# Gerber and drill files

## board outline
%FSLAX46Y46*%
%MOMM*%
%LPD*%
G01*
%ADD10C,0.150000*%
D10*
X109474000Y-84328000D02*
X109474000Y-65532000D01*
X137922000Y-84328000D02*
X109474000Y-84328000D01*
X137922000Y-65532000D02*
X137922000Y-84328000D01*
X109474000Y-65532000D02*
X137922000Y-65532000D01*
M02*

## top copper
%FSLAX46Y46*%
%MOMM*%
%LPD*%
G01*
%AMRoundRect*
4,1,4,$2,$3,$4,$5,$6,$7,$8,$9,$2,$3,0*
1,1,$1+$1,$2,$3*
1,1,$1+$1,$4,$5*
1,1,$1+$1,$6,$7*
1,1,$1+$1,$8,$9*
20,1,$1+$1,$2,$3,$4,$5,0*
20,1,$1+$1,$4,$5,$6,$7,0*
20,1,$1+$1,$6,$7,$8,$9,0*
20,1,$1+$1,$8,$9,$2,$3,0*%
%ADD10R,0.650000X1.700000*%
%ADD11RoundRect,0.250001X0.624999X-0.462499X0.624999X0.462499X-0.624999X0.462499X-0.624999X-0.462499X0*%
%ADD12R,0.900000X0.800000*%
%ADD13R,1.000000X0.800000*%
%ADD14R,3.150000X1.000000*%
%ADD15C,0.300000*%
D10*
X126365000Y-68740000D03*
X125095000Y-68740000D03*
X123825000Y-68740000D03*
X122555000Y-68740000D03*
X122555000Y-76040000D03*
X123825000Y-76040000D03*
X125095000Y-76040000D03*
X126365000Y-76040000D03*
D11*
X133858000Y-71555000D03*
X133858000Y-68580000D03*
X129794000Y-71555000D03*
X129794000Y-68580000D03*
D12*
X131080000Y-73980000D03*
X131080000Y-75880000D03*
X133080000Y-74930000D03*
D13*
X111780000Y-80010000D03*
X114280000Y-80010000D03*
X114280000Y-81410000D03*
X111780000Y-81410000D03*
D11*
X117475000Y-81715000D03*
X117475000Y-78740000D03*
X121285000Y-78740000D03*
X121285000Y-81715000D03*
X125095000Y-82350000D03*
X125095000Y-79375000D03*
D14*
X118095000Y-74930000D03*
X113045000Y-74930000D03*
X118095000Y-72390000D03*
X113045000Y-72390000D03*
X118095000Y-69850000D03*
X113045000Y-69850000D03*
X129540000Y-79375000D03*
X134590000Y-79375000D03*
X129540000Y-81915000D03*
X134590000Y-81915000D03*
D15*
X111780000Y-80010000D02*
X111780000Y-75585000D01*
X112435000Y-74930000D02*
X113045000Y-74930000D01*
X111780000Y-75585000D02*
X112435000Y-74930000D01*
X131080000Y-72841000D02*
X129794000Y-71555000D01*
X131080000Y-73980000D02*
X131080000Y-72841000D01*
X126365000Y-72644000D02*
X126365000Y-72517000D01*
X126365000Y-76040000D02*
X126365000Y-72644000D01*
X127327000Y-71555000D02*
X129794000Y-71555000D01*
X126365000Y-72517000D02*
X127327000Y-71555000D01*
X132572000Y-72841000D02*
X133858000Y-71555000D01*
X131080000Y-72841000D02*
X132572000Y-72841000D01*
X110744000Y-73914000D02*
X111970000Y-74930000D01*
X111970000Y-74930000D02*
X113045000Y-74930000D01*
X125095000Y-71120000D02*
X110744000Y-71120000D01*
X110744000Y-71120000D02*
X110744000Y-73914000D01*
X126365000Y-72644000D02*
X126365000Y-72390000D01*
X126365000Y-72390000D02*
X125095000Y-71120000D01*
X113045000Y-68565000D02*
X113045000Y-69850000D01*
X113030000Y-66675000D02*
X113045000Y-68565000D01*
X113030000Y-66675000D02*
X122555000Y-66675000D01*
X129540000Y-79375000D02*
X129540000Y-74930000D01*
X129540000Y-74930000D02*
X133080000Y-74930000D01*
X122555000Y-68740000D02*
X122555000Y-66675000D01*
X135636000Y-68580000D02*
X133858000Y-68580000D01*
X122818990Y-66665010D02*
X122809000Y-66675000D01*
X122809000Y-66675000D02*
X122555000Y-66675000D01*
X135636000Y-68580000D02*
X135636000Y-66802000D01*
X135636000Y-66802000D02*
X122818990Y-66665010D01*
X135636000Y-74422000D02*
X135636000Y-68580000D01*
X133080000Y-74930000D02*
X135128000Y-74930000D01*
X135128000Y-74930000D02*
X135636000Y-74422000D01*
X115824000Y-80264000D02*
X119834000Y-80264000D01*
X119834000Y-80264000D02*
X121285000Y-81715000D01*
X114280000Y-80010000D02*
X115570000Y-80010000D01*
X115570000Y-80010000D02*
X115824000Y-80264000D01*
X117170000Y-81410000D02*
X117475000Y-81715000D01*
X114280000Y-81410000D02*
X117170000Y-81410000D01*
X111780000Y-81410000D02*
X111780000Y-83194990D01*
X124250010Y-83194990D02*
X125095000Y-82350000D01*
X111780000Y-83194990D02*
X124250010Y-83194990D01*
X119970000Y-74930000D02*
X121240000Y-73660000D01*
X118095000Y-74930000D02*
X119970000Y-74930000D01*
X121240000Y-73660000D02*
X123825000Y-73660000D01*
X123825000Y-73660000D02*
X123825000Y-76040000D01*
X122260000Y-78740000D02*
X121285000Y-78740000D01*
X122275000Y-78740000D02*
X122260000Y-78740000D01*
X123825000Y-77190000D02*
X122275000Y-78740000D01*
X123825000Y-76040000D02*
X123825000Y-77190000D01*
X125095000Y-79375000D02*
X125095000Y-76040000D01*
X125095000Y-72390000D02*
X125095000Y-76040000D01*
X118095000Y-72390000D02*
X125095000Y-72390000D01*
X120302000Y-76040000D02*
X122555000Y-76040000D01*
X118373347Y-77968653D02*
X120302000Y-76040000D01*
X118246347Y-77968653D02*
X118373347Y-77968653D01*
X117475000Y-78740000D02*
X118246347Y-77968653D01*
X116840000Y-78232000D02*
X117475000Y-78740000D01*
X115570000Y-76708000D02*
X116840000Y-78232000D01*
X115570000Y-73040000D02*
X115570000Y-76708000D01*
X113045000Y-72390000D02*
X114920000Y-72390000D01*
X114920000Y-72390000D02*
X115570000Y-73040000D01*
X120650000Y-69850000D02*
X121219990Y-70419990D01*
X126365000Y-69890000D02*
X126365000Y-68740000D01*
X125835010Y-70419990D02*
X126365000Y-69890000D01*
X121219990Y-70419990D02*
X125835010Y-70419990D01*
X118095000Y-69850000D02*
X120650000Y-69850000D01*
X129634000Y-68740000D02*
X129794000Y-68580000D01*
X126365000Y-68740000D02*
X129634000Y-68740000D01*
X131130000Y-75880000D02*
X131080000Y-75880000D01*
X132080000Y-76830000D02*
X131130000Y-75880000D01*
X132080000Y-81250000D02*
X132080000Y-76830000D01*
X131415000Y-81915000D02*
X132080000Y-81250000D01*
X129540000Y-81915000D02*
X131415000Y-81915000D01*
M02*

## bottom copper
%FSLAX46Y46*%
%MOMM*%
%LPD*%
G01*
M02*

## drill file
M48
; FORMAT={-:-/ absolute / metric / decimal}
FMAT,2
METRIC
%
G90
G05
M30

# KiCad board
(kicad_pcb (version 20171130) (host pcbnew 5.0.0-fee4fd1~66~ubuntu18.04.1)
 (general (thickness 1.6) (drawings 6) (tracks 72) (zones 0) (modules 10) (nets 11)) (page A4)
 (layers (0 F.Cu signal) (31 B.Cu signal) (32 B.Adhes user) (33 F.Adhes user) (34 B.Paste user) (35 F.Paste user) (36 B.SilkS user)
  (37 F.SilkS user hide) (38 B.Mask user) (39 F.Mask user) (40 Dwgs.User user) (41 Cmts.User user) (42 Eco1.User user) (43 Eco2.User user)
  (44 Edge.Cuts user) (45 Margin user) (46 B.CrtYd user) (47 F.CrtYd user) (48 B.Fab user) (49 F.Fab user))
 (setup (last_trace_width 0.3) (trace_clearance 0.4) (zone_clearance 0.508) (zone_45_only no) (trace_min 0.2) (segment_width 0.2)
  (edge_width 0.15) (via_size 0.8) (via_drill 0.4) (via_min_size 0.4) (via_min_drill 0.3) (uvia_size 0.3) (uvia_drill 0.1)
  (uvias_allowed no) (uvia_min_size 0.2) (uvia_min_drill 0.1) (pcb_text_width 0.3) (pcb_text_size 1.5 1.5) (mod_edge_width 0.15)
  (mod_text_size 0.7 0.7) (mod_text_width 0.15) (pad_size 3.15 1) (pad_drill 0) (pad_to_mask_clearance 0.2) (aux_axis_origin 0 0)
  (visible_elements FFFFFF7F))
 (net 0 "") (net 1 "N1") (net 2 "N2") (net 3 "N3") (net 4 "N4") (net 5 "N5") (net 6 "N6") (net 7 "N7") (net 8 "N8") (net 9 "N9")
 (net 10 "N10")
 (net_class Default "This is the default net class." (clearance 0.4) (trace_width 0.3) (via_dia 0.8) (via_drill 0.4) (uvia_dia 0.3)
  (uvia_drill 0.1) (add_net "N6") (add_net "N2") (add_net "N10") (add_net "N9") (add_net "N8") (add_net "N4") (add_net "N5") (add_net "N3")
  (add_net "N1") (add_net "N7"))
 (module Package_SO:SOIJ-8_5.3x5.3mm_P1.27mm (layer F.Cu) (at 124.46 72.39 270)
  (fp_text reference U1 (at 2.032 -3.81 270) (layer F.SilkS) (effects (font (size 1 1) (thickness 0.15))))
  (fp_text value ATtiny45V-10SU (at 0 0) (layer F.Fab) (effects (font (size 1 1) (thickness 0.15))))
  (pad 1 smd rect (at -3.65 -1.905 270) (size 1.7 0.65) (layers F.Cu F.Paste F.Mask) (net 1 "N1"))
  (pad 2 smd rect (at -3.65 -0.635 270) (size 1.7 0.65) (layers F.Cu F.Paste F.Mask))
  (pad 3 smd rect (at -3.65 0.635 270) (size 1.7 0.65) (layers F.Cu F.Paste F.Mask))
  (pad 4 smd rect (at -3.65 1.905 270) (size 1.7 0.65) (layers F.Cu F.Paste F.Mask) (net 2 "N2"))
  (pad 5 smd rect (at 3.65 1.905 270) (size 1.7 0.65) (layers F.Cu F.Paste F.Mask) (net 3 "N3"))
  (pad 6 smd rect (at 3.65 0.635 270) (size 1.7 0.65) (layers F.Cu F.Paste F.Mask) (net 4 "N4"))
  (pad 7 smd rect (at 3.65 -0.635 270) (size 1.7 0.65) (layers F.Cu F.Paste F.Mask) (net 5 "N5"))
  (pad 8 smd rect (at 3.65 -1.905 270) (size 1.7 0.65) (layers F.Cu F.Paste F.Mask) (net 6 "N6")))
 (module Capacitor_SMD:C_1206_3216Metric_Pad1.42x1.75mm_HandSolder (layer F.Cu) (at 133.858 70.0675 90)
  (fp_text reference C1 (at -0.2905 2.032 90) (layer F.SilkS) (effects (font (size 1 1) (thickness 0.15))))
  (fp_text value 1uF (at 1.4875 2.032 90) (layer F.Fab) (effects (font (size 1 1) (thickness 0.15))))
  (pad 1 smd roundrect (at -1.4875 0 90) (size 1.425 1.75) (layers F.Cu F.Paste F.Mask) (roundrect_rratio 0.175439) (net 6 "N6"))
  (pad 2 smd roundrect (at 1.4875 0 90) (size 1.425 1.75) (layers F.Cu F.Paste F.Mask) (roundrect_rratio 0.175439) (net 2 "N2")))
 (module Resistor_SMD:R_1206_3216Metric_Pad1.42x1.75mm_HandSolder (layer F.Cu) (at 129.794 70.0675 90)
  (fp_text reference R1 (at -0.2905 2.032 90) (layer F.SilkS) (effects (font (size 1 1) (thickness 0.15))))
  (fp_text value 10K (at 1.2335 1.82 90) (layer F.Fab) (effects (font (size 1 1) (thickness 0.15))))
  (pad 1 smd roundrect (at -1.4875 0 90) (size 1.425 1.75) (layers F.Cu F.Paste F.Mask) (roundrect_rratio 0.175439) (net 6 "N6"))
  (pad 2 smd roundrect (at 1.4875 0 90) (size 1.425 1.75) (layers F.Cu F.Paste F.Mask) (roundrect_rratio 0.175439) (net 1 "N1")))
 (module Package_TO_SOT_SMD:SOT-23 (layer F.Cu) (at 132.08 74.93)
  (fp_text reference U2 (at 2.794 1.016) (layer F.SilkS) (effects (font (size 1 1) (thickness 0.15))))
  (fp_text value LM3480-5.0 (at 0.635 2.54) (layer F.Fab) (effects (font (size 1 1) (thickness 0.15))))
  (pad 1 smd rect (at -1 -0.95) (size 0.9 0.8) (layers F.Cu F.Paste F.Mask) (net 6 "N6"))
  (pad 2 smd rect (at -1 0.95) (size 0.9 0.8) (layers F.Cu F.Paste F.Mask) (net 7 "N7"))
  (pad 3 smd rect (at 1 0) (size 0.9 0.8) (layers F.Cu F.Paste F.Mask) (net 2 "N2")))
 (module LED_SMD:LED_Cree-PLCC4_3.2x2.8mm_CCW (layer F.Cu) (at 113.03 80.71)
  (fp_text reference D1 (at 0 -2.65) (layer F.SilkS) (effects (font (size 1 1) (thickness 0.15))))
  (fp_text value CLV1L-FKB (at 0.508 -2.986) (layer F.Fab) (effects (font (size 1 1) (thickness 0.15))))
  (pad 1 smd rect (at -1.25 -0.7) (size 1 0.8) (layers F.Cu F.Paste F.Mask) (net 6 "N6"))
  (pad 4 smd rect (at 1.25 -0.7) (size 1 0.8) (layers F.Cu F.Paste F.Mask) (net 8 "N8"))
  (pad 3 smd rect (at 1.25 0.7) (size 1 0.8) (layers F.Cu F.Paste F.Mask) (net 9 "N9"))
  (pad 2 smd rect (at -1.25 0.7) (size 1 0.8) (layers F.Cu F.Paste F.Mask) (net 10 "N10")))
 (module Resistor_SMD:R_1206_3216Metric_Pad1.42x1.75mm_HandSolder (layer F.Cu) (at 117.475 80.2275 90)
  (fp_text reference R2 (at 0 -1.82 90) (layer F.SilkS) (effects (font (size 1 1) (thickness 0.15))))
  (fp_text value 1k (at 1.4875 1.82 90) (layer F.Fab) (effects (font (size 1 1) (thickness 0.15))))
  (pad 1 smd roundrect (at -1.4875 0 90) (size 1.425 1.75) (layers F.Cu F.Paste F.Mask) (roundrect_rratio 0.175439) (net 9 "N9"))
  (pad 2 smd roundrect (at 1.4875 0 90) (size 1.425 1.75) (layers F.Cu F.Paste F.Mask) (roundrect_rratio 0.175439) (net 3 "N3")))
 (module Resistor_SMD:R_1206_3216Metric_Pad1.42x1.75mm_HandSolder (layer F.Cu) (at 121.285 80.2275 90)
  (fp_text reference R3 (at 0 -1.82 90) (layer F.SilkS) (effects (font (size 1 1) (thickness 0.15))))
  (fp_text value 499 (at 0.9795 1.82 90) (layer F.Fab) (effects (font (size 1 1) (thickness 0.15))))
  (pad 2 smd roundrect (at 1.4875 0 90) (size 1.425 1.75) (layers F.Cu F.Paste F.Mask) (roundrect_rratio 0.175439) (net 4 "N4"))
  (pad 1 smd roundrect (at -1.4875 0 90) (size 1.425 1.75) (layers F.Cu F.Paste F.Mask) (roundrect_rratio 0.175439) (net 8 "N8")))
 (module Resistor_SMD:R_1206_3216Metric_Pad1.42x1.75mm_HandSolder (layer F.Cu) (at 125.095 80.8625 90)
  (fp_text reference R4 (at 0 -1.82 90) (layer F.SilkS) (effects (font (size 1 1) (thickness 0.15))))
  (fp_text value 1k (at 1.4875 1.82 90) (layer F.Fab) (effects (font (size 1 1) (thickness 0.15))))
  (pad 1 smd roundrect (at -1.4875 0 90) (size 1.425 1.75) (layers F.Cu F.Paste F.Mask) (roundrect_rratio 0.175439) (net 10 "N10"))
  (pad 2 smd roundrect (at 1.4875 0 90) (size 1.425 1.75) (layers F.Cu F.Paste F.Mask) (roundrect_rratio 0.175439) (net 5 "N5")))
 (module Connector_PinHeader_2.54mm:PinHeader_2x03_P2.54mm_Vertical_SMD (layer F.Cu) (at 115.57 72.39 180)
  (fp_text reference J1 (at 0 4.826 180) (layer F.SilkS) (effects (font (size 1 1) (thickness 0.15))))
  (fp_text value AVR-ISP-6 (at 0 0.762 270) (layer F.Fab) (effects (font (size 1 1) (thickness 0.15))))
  (pad 1 smd rect (at -2.525 -2.54 180) (size 3.15 1) (layers F.Cu F.Paste F.Mask) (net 4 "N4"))
  (pad 2 smd rect (at 2.525 -2.54 180) (size 3.15 1) (layers F.Cu F.Paste F.Mask) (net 6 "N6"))
  (pad 3 smd rect (at -2.525 0 180) (size 3.15 1) (layers F.Cu F.Paste F.Mask) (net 5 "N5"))
  (pad 4 smd rect (at 2.525 0 180) (size 3.15 1) (layers F.Cu F.Paste F.Mask) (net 3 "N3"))
  (pad 5 smd rect (at -2.525 2.54 180) (size 3.15 1) (layers F.Cu F.Paste F.Mask) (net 1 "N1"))
  (pad 6 smd rect (at 2.525 2.54 180) (size 3.15 1) (layers F.Cu F.Paste F.Mask) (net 2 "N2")))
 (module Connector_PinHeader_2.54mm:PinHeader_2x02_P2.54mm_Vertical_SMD (layer F.Cu) (at 132.065 80.645)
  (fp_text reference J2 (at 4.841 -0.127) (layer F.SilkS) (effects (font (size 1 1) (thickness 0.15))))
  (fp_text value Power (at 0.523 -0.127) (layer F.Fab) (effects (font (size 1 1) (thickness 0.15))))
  (pad 1 smd rect (at -2.525 -1.27) (size 3.15 1) (layers F.Cu F.Paste F.Mask) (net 2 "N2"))
  (pad 2 smd rect (at 2.525 -1.27) (size 3.15 1) (layers F.Cu F.Paste F.Mask))
  (pad 3 smd rect (at -2.525 1.27) (size 3.15 1) (layers F.Cu F.Paste F.Mask) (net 7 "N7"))
  (pad 4 smd rect (at 2.525 1.27) (size 3.15 1) (layers F.Cu F.Paste F.Mask)))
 (gr_line (start 109.474 84.328) (end 109.474 65.532) (layer Edge.Cuts) (width 0.15))
 (gr_line (start 137.922 84.328) (end 109.474 84.328) (layer Edge.Cuts) (width 0.15))
 (gr_line (start 137.922 65.532) (end 137.922 84.328) (layer Edge.Cuts) (width 0.15))
 (gr_line (start 109.474 65.532) (end 137.922 65.532) (layer Edge.Cuts) (width 0.15))
 (segment (start 111.78 80.01) (end 111.78 75.585) (width 0.3) (layer F.Cu) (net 6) (status 10))
 (segment (start 112.435 74.93) (end 113.045 74.93) (width 0.3) (layer F.Cu) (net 6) (status 30))
 (segment (start 111.78 75.585) (end 112.435 74.93) (width 0.3) (layer F.Cu) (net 6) (status 20))
 (segment (start 131.08 72.841) (end 129.794 71.555) (width 0.3) (layer F.Cu) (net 6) (status 20))
 (segment (start 131.08 73.98) (end 131.08 72.841) (width 0.3) (layer F.Cu) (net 6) (status 10))
 (segment (start 126.365 72.644) (end 126.365 72.517) (width 0.3) (layer F.Cu) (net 6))
 (segment (start 126.365 76.04) (end 126.365 72.644) (width 0.3) (layer F.Cu) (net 6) (status 10))
 (segment (start 127.327 71.555) (end 129.794 71.555) (width 0.3) (layer F.Cu) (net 6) (status 20))
 (segment (start 126.365 72.517) (end 127.327 71.555) (width 0.3) (layer F.Cu) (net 6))
 (segment (start 132.572 72.841) (end 133.858 71.555) (width 0.3) (layer F.Cu) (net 6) (status 20))
 (segment (start 131.08 72.841) (end 132.572 72.841) (width 0.3) (layer F.Cu) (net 6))
 (segment (start 110.744 73.914) (end 111.97 74.93) (width 0.3) (layer F.Cu) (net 6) (status 20))
 (segment (start 111.97 74.93) (end 113.045 74.93) (width 0.3) (layer F.Cu) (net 6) (status 30))
 (segment (start 125.095 71.12) (end 110.744 71.12) (width 0.3) (layer F.Cu) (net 6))
 (segment (start 110.744 71.12) (end 110.744 73.914) (width 0.3) (layer F.Cu) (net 6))
 (segment (start 126.365 72.644) (end 126.365 72.39) (width 0.3) (layer F.Cu) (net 6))
 (segment (start 126.365 72.39) (end 125.095 71.12) (width 0.3) (layer F.Cu) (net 6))
 (segment (start 113.045 68.565) (end 113.045 69.85) (width 0.3) (layer F.Cu) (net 2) (status 20))
 (segment (start 113.03 66.675) (end 113.045 68.565) (width 0.3) (layer F.Cu) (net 2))
 (segment (start 113.03 66.675) (end 122.555 66.675) (width 0.3) (layer F.Cu) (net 2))
 (segment (start 129.54 79.375) (end 129.54 74.93) (width 0.3) (layer F.Cu) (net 2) (status 10))
 (segment (start 129.54 74.93) (end 133.08 74.93) (width 0.3) (layer F.Cu) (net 2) (status 20))
 (segment (start 122.555 68.74) (end 122.555 66.675) (width 0.3) (layer F.Cu) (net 2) (status 10))
 (segment (start 135.636 68.58) (end 133.858 68.58) (width 0.3) (layer F.Cu) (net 2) (status 20))
 (segment (start 122.81899 66.66501) (end 122.809 66.675) (width 0.3) (layer F.Cu) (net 2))
 (segment (start 122.809 66.675) (end 122.555 66.675) (width 0.3) (layer F.Cu) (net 2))
 (segment (start 135.636 68.58) (end 135.636 66.802) (width 0.3) (layer F.Cu) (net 2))
 (segment (start 135.636 66.802) (end 122.81899 66.66501) (width 0.3) (layer F.Cu) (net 2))
 (segment (start 135.636 74.422) (end 135.636 68.58) (width 0.3) (layer F.Cu) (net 2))
 (segment (start 133.08 74.93) (end 135.128 74.93) (width 0.3) (layer F.Cu) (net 2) (status 10))
 (segment (start 135.128 74.93) (end 135.636 74.422) (width 0.3) (layer F.Cu) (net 2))
 (segment (start 115.824 80.264) (end 119.834 80.264) (width 0.3) (layer F.Cu) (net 8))
 (segment (start 119.834 80.264) (end 121.285 81.715) (width 0.3) (layer F.Cu) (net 8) (status 20))
 (segment (start 114.28 80.01) (end 115.57 80.01) (width 0.3) (layer F.Cu) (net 8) (status 10))
 (segment (start 115.57 80.01) (end 115.824 80.264) (width 0.3) (layer F.Cu) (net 8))
 (segment (start 117.17 81.41) (end 117.475 81.715) (width 0.3) (layer F.Cu) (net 9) (status 30))
 (segment (start 114.28 81.41) (end 117.17 81.41) (width 0.3) (layer F.Cu) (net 9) (status 30))
 (segment (start 111.78 81.41) (end 111.78 83.19499) (width 0.3) (layer F.Cu) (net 10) (status 10))
 (segment (start 124.25001 83.19499) (end 125.095 82.35) (width 0.3) (layer F.Cu) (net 10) (status 20))
 (segment (start 111.78 83.19499) (end 124.25001 83.19499) (width 0.3) (layer F.Cu) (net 10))
 (segment (start 119.97 74.93) (end 121.24 73.66) (width 0.3) (layer F.Cu) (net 4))
 (segment (start 118.095 74.93) (end 119.97 74.93) (width 0.3) (layer F.Cu) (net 4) (status 10))
 (segment (start 121.24 73.66) (end 123.825 73.66) (width 0.3) (layer F.Cu) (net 4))
 (segment (start 123.825 73.66) (end 123.825 76.04) (width 0.3) (layer F.Cu) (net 4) (status 20))
 (segment (start 122.26 78.74) (end 121.285 78.74) (width 0.3) (layer F.Cu) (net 4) (status 20))
 (segment (start 122.275 78.74) (end 122.26 78.74) (width 0.3) (layer F.Cu) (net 4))
 (segment (start 123.825 77.19) (end 122.275 78.74) (width 0.3) (layer F.Cu) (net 4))
 (segment (start 123.825 76.04) (end 123.825 77.19) (width 0.3) (layer F.Cu) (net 4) (status 10))
 (segment (start 125.095 79.375) (end 125.095 76.04) (width 0.3) (layer F.Cu) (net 5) (status 30))
 (segment (start 125.095 72.39) (end 125.095 76.04) (width 0.3) (layer F.Cu) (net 5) (status 20))
 (segment (start 118.095 72.39) (end 125.095 72.39) (width 0.3) (layer F.Cu) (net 5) (status 10))
 (segment (start 120.302 76.04) (end 122.555 76.04) (width 0.3) (layer F.Cu) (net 3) (status 20))
 (segment (start 118.373347 77.968653) (end 120.302 76.04) (width 0.3) (layer F.Cu) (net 3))
 (segment (start 118.246347 77.968653) (end 118.373347 77.968653) (width 0.3) (layer F.Cu) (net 3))
 (segment (start 117.475 78.74) (end 118.246347 77.968653) (width 0.3) (layer F.Cu) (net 3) (status 10))
 (segment (start 116.84 78.232) (end 117.475 78.74) (width 0.3) (layer F.Cu) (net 3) (status 30))
 (segment (start 115.57 76.708) (end 116.84 78.232) (width 0.3) (layer F.Cu) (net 3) (status 20))
 (segment (start 115.57 73.04) (end 115.57 76.708) (width 0.3) (layer F.Cu) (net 3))
 (segment (start 113.045 72.39) (end 114.92 72.39) (width 0.3) (layer F.Cu) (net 3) (status 10))
 (segment (start 114.92 72.39) (end 115.57 73.04) (width 0.3) (layer F.Cu) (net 3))
 (segment (start 120.65 69.85) (end 121.21999 70.41999) (width 0.3) (layer F.Cu) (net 1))
 (segment (start 126.365 69.89) (end 126.365 68.74) (width 0.3) (layer F.Cu) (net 1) (status 20))
 (segment (start 125.83501 70.41999) (end 126.365 69.89) (width 0.3) (layer F.Cu) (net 1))
 (segment (start 121.21999 70.41999) (end 125.83501 70.41999) (width 0.3) (layer F.Cu) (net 1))
 (segment (start 118.095 69.85) (end 120.65 69.85) (width 0.3) (layer F.Cu) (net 1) (status 10))
 (segment (start 129.634 68.74) (end 129.794 68.58) (width 0.3) (layer F.Cu) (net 1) (status 30))
 (segment (start 126.365 68.74) (end 129.634 68.74) (width 0.3) (layer F.Cu) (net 1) (status 30))
 (segment (start 131.13 75.88) (end 131.08 75.88) (width 0.3) (layer F.Cu) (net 7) (status 30))
 (segment (start 132.08 76.83) (end 131.13 75.88) (width 0.3) (layer F.Cu) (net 7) (status 20))
 (segment (start 132.08 81.25) (end 132.08 76.83) (width 0.3) (layer F.Cu) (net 7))
 (segment (start 131.415 81.915) (end 132.08 81.25) (width 0.3) (layer F.Cu) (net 7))
 (segment (start 129.54 81.915) (end 131.415 81.915) (width 0.3) (layer F.Cu) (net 7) (status 10)))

